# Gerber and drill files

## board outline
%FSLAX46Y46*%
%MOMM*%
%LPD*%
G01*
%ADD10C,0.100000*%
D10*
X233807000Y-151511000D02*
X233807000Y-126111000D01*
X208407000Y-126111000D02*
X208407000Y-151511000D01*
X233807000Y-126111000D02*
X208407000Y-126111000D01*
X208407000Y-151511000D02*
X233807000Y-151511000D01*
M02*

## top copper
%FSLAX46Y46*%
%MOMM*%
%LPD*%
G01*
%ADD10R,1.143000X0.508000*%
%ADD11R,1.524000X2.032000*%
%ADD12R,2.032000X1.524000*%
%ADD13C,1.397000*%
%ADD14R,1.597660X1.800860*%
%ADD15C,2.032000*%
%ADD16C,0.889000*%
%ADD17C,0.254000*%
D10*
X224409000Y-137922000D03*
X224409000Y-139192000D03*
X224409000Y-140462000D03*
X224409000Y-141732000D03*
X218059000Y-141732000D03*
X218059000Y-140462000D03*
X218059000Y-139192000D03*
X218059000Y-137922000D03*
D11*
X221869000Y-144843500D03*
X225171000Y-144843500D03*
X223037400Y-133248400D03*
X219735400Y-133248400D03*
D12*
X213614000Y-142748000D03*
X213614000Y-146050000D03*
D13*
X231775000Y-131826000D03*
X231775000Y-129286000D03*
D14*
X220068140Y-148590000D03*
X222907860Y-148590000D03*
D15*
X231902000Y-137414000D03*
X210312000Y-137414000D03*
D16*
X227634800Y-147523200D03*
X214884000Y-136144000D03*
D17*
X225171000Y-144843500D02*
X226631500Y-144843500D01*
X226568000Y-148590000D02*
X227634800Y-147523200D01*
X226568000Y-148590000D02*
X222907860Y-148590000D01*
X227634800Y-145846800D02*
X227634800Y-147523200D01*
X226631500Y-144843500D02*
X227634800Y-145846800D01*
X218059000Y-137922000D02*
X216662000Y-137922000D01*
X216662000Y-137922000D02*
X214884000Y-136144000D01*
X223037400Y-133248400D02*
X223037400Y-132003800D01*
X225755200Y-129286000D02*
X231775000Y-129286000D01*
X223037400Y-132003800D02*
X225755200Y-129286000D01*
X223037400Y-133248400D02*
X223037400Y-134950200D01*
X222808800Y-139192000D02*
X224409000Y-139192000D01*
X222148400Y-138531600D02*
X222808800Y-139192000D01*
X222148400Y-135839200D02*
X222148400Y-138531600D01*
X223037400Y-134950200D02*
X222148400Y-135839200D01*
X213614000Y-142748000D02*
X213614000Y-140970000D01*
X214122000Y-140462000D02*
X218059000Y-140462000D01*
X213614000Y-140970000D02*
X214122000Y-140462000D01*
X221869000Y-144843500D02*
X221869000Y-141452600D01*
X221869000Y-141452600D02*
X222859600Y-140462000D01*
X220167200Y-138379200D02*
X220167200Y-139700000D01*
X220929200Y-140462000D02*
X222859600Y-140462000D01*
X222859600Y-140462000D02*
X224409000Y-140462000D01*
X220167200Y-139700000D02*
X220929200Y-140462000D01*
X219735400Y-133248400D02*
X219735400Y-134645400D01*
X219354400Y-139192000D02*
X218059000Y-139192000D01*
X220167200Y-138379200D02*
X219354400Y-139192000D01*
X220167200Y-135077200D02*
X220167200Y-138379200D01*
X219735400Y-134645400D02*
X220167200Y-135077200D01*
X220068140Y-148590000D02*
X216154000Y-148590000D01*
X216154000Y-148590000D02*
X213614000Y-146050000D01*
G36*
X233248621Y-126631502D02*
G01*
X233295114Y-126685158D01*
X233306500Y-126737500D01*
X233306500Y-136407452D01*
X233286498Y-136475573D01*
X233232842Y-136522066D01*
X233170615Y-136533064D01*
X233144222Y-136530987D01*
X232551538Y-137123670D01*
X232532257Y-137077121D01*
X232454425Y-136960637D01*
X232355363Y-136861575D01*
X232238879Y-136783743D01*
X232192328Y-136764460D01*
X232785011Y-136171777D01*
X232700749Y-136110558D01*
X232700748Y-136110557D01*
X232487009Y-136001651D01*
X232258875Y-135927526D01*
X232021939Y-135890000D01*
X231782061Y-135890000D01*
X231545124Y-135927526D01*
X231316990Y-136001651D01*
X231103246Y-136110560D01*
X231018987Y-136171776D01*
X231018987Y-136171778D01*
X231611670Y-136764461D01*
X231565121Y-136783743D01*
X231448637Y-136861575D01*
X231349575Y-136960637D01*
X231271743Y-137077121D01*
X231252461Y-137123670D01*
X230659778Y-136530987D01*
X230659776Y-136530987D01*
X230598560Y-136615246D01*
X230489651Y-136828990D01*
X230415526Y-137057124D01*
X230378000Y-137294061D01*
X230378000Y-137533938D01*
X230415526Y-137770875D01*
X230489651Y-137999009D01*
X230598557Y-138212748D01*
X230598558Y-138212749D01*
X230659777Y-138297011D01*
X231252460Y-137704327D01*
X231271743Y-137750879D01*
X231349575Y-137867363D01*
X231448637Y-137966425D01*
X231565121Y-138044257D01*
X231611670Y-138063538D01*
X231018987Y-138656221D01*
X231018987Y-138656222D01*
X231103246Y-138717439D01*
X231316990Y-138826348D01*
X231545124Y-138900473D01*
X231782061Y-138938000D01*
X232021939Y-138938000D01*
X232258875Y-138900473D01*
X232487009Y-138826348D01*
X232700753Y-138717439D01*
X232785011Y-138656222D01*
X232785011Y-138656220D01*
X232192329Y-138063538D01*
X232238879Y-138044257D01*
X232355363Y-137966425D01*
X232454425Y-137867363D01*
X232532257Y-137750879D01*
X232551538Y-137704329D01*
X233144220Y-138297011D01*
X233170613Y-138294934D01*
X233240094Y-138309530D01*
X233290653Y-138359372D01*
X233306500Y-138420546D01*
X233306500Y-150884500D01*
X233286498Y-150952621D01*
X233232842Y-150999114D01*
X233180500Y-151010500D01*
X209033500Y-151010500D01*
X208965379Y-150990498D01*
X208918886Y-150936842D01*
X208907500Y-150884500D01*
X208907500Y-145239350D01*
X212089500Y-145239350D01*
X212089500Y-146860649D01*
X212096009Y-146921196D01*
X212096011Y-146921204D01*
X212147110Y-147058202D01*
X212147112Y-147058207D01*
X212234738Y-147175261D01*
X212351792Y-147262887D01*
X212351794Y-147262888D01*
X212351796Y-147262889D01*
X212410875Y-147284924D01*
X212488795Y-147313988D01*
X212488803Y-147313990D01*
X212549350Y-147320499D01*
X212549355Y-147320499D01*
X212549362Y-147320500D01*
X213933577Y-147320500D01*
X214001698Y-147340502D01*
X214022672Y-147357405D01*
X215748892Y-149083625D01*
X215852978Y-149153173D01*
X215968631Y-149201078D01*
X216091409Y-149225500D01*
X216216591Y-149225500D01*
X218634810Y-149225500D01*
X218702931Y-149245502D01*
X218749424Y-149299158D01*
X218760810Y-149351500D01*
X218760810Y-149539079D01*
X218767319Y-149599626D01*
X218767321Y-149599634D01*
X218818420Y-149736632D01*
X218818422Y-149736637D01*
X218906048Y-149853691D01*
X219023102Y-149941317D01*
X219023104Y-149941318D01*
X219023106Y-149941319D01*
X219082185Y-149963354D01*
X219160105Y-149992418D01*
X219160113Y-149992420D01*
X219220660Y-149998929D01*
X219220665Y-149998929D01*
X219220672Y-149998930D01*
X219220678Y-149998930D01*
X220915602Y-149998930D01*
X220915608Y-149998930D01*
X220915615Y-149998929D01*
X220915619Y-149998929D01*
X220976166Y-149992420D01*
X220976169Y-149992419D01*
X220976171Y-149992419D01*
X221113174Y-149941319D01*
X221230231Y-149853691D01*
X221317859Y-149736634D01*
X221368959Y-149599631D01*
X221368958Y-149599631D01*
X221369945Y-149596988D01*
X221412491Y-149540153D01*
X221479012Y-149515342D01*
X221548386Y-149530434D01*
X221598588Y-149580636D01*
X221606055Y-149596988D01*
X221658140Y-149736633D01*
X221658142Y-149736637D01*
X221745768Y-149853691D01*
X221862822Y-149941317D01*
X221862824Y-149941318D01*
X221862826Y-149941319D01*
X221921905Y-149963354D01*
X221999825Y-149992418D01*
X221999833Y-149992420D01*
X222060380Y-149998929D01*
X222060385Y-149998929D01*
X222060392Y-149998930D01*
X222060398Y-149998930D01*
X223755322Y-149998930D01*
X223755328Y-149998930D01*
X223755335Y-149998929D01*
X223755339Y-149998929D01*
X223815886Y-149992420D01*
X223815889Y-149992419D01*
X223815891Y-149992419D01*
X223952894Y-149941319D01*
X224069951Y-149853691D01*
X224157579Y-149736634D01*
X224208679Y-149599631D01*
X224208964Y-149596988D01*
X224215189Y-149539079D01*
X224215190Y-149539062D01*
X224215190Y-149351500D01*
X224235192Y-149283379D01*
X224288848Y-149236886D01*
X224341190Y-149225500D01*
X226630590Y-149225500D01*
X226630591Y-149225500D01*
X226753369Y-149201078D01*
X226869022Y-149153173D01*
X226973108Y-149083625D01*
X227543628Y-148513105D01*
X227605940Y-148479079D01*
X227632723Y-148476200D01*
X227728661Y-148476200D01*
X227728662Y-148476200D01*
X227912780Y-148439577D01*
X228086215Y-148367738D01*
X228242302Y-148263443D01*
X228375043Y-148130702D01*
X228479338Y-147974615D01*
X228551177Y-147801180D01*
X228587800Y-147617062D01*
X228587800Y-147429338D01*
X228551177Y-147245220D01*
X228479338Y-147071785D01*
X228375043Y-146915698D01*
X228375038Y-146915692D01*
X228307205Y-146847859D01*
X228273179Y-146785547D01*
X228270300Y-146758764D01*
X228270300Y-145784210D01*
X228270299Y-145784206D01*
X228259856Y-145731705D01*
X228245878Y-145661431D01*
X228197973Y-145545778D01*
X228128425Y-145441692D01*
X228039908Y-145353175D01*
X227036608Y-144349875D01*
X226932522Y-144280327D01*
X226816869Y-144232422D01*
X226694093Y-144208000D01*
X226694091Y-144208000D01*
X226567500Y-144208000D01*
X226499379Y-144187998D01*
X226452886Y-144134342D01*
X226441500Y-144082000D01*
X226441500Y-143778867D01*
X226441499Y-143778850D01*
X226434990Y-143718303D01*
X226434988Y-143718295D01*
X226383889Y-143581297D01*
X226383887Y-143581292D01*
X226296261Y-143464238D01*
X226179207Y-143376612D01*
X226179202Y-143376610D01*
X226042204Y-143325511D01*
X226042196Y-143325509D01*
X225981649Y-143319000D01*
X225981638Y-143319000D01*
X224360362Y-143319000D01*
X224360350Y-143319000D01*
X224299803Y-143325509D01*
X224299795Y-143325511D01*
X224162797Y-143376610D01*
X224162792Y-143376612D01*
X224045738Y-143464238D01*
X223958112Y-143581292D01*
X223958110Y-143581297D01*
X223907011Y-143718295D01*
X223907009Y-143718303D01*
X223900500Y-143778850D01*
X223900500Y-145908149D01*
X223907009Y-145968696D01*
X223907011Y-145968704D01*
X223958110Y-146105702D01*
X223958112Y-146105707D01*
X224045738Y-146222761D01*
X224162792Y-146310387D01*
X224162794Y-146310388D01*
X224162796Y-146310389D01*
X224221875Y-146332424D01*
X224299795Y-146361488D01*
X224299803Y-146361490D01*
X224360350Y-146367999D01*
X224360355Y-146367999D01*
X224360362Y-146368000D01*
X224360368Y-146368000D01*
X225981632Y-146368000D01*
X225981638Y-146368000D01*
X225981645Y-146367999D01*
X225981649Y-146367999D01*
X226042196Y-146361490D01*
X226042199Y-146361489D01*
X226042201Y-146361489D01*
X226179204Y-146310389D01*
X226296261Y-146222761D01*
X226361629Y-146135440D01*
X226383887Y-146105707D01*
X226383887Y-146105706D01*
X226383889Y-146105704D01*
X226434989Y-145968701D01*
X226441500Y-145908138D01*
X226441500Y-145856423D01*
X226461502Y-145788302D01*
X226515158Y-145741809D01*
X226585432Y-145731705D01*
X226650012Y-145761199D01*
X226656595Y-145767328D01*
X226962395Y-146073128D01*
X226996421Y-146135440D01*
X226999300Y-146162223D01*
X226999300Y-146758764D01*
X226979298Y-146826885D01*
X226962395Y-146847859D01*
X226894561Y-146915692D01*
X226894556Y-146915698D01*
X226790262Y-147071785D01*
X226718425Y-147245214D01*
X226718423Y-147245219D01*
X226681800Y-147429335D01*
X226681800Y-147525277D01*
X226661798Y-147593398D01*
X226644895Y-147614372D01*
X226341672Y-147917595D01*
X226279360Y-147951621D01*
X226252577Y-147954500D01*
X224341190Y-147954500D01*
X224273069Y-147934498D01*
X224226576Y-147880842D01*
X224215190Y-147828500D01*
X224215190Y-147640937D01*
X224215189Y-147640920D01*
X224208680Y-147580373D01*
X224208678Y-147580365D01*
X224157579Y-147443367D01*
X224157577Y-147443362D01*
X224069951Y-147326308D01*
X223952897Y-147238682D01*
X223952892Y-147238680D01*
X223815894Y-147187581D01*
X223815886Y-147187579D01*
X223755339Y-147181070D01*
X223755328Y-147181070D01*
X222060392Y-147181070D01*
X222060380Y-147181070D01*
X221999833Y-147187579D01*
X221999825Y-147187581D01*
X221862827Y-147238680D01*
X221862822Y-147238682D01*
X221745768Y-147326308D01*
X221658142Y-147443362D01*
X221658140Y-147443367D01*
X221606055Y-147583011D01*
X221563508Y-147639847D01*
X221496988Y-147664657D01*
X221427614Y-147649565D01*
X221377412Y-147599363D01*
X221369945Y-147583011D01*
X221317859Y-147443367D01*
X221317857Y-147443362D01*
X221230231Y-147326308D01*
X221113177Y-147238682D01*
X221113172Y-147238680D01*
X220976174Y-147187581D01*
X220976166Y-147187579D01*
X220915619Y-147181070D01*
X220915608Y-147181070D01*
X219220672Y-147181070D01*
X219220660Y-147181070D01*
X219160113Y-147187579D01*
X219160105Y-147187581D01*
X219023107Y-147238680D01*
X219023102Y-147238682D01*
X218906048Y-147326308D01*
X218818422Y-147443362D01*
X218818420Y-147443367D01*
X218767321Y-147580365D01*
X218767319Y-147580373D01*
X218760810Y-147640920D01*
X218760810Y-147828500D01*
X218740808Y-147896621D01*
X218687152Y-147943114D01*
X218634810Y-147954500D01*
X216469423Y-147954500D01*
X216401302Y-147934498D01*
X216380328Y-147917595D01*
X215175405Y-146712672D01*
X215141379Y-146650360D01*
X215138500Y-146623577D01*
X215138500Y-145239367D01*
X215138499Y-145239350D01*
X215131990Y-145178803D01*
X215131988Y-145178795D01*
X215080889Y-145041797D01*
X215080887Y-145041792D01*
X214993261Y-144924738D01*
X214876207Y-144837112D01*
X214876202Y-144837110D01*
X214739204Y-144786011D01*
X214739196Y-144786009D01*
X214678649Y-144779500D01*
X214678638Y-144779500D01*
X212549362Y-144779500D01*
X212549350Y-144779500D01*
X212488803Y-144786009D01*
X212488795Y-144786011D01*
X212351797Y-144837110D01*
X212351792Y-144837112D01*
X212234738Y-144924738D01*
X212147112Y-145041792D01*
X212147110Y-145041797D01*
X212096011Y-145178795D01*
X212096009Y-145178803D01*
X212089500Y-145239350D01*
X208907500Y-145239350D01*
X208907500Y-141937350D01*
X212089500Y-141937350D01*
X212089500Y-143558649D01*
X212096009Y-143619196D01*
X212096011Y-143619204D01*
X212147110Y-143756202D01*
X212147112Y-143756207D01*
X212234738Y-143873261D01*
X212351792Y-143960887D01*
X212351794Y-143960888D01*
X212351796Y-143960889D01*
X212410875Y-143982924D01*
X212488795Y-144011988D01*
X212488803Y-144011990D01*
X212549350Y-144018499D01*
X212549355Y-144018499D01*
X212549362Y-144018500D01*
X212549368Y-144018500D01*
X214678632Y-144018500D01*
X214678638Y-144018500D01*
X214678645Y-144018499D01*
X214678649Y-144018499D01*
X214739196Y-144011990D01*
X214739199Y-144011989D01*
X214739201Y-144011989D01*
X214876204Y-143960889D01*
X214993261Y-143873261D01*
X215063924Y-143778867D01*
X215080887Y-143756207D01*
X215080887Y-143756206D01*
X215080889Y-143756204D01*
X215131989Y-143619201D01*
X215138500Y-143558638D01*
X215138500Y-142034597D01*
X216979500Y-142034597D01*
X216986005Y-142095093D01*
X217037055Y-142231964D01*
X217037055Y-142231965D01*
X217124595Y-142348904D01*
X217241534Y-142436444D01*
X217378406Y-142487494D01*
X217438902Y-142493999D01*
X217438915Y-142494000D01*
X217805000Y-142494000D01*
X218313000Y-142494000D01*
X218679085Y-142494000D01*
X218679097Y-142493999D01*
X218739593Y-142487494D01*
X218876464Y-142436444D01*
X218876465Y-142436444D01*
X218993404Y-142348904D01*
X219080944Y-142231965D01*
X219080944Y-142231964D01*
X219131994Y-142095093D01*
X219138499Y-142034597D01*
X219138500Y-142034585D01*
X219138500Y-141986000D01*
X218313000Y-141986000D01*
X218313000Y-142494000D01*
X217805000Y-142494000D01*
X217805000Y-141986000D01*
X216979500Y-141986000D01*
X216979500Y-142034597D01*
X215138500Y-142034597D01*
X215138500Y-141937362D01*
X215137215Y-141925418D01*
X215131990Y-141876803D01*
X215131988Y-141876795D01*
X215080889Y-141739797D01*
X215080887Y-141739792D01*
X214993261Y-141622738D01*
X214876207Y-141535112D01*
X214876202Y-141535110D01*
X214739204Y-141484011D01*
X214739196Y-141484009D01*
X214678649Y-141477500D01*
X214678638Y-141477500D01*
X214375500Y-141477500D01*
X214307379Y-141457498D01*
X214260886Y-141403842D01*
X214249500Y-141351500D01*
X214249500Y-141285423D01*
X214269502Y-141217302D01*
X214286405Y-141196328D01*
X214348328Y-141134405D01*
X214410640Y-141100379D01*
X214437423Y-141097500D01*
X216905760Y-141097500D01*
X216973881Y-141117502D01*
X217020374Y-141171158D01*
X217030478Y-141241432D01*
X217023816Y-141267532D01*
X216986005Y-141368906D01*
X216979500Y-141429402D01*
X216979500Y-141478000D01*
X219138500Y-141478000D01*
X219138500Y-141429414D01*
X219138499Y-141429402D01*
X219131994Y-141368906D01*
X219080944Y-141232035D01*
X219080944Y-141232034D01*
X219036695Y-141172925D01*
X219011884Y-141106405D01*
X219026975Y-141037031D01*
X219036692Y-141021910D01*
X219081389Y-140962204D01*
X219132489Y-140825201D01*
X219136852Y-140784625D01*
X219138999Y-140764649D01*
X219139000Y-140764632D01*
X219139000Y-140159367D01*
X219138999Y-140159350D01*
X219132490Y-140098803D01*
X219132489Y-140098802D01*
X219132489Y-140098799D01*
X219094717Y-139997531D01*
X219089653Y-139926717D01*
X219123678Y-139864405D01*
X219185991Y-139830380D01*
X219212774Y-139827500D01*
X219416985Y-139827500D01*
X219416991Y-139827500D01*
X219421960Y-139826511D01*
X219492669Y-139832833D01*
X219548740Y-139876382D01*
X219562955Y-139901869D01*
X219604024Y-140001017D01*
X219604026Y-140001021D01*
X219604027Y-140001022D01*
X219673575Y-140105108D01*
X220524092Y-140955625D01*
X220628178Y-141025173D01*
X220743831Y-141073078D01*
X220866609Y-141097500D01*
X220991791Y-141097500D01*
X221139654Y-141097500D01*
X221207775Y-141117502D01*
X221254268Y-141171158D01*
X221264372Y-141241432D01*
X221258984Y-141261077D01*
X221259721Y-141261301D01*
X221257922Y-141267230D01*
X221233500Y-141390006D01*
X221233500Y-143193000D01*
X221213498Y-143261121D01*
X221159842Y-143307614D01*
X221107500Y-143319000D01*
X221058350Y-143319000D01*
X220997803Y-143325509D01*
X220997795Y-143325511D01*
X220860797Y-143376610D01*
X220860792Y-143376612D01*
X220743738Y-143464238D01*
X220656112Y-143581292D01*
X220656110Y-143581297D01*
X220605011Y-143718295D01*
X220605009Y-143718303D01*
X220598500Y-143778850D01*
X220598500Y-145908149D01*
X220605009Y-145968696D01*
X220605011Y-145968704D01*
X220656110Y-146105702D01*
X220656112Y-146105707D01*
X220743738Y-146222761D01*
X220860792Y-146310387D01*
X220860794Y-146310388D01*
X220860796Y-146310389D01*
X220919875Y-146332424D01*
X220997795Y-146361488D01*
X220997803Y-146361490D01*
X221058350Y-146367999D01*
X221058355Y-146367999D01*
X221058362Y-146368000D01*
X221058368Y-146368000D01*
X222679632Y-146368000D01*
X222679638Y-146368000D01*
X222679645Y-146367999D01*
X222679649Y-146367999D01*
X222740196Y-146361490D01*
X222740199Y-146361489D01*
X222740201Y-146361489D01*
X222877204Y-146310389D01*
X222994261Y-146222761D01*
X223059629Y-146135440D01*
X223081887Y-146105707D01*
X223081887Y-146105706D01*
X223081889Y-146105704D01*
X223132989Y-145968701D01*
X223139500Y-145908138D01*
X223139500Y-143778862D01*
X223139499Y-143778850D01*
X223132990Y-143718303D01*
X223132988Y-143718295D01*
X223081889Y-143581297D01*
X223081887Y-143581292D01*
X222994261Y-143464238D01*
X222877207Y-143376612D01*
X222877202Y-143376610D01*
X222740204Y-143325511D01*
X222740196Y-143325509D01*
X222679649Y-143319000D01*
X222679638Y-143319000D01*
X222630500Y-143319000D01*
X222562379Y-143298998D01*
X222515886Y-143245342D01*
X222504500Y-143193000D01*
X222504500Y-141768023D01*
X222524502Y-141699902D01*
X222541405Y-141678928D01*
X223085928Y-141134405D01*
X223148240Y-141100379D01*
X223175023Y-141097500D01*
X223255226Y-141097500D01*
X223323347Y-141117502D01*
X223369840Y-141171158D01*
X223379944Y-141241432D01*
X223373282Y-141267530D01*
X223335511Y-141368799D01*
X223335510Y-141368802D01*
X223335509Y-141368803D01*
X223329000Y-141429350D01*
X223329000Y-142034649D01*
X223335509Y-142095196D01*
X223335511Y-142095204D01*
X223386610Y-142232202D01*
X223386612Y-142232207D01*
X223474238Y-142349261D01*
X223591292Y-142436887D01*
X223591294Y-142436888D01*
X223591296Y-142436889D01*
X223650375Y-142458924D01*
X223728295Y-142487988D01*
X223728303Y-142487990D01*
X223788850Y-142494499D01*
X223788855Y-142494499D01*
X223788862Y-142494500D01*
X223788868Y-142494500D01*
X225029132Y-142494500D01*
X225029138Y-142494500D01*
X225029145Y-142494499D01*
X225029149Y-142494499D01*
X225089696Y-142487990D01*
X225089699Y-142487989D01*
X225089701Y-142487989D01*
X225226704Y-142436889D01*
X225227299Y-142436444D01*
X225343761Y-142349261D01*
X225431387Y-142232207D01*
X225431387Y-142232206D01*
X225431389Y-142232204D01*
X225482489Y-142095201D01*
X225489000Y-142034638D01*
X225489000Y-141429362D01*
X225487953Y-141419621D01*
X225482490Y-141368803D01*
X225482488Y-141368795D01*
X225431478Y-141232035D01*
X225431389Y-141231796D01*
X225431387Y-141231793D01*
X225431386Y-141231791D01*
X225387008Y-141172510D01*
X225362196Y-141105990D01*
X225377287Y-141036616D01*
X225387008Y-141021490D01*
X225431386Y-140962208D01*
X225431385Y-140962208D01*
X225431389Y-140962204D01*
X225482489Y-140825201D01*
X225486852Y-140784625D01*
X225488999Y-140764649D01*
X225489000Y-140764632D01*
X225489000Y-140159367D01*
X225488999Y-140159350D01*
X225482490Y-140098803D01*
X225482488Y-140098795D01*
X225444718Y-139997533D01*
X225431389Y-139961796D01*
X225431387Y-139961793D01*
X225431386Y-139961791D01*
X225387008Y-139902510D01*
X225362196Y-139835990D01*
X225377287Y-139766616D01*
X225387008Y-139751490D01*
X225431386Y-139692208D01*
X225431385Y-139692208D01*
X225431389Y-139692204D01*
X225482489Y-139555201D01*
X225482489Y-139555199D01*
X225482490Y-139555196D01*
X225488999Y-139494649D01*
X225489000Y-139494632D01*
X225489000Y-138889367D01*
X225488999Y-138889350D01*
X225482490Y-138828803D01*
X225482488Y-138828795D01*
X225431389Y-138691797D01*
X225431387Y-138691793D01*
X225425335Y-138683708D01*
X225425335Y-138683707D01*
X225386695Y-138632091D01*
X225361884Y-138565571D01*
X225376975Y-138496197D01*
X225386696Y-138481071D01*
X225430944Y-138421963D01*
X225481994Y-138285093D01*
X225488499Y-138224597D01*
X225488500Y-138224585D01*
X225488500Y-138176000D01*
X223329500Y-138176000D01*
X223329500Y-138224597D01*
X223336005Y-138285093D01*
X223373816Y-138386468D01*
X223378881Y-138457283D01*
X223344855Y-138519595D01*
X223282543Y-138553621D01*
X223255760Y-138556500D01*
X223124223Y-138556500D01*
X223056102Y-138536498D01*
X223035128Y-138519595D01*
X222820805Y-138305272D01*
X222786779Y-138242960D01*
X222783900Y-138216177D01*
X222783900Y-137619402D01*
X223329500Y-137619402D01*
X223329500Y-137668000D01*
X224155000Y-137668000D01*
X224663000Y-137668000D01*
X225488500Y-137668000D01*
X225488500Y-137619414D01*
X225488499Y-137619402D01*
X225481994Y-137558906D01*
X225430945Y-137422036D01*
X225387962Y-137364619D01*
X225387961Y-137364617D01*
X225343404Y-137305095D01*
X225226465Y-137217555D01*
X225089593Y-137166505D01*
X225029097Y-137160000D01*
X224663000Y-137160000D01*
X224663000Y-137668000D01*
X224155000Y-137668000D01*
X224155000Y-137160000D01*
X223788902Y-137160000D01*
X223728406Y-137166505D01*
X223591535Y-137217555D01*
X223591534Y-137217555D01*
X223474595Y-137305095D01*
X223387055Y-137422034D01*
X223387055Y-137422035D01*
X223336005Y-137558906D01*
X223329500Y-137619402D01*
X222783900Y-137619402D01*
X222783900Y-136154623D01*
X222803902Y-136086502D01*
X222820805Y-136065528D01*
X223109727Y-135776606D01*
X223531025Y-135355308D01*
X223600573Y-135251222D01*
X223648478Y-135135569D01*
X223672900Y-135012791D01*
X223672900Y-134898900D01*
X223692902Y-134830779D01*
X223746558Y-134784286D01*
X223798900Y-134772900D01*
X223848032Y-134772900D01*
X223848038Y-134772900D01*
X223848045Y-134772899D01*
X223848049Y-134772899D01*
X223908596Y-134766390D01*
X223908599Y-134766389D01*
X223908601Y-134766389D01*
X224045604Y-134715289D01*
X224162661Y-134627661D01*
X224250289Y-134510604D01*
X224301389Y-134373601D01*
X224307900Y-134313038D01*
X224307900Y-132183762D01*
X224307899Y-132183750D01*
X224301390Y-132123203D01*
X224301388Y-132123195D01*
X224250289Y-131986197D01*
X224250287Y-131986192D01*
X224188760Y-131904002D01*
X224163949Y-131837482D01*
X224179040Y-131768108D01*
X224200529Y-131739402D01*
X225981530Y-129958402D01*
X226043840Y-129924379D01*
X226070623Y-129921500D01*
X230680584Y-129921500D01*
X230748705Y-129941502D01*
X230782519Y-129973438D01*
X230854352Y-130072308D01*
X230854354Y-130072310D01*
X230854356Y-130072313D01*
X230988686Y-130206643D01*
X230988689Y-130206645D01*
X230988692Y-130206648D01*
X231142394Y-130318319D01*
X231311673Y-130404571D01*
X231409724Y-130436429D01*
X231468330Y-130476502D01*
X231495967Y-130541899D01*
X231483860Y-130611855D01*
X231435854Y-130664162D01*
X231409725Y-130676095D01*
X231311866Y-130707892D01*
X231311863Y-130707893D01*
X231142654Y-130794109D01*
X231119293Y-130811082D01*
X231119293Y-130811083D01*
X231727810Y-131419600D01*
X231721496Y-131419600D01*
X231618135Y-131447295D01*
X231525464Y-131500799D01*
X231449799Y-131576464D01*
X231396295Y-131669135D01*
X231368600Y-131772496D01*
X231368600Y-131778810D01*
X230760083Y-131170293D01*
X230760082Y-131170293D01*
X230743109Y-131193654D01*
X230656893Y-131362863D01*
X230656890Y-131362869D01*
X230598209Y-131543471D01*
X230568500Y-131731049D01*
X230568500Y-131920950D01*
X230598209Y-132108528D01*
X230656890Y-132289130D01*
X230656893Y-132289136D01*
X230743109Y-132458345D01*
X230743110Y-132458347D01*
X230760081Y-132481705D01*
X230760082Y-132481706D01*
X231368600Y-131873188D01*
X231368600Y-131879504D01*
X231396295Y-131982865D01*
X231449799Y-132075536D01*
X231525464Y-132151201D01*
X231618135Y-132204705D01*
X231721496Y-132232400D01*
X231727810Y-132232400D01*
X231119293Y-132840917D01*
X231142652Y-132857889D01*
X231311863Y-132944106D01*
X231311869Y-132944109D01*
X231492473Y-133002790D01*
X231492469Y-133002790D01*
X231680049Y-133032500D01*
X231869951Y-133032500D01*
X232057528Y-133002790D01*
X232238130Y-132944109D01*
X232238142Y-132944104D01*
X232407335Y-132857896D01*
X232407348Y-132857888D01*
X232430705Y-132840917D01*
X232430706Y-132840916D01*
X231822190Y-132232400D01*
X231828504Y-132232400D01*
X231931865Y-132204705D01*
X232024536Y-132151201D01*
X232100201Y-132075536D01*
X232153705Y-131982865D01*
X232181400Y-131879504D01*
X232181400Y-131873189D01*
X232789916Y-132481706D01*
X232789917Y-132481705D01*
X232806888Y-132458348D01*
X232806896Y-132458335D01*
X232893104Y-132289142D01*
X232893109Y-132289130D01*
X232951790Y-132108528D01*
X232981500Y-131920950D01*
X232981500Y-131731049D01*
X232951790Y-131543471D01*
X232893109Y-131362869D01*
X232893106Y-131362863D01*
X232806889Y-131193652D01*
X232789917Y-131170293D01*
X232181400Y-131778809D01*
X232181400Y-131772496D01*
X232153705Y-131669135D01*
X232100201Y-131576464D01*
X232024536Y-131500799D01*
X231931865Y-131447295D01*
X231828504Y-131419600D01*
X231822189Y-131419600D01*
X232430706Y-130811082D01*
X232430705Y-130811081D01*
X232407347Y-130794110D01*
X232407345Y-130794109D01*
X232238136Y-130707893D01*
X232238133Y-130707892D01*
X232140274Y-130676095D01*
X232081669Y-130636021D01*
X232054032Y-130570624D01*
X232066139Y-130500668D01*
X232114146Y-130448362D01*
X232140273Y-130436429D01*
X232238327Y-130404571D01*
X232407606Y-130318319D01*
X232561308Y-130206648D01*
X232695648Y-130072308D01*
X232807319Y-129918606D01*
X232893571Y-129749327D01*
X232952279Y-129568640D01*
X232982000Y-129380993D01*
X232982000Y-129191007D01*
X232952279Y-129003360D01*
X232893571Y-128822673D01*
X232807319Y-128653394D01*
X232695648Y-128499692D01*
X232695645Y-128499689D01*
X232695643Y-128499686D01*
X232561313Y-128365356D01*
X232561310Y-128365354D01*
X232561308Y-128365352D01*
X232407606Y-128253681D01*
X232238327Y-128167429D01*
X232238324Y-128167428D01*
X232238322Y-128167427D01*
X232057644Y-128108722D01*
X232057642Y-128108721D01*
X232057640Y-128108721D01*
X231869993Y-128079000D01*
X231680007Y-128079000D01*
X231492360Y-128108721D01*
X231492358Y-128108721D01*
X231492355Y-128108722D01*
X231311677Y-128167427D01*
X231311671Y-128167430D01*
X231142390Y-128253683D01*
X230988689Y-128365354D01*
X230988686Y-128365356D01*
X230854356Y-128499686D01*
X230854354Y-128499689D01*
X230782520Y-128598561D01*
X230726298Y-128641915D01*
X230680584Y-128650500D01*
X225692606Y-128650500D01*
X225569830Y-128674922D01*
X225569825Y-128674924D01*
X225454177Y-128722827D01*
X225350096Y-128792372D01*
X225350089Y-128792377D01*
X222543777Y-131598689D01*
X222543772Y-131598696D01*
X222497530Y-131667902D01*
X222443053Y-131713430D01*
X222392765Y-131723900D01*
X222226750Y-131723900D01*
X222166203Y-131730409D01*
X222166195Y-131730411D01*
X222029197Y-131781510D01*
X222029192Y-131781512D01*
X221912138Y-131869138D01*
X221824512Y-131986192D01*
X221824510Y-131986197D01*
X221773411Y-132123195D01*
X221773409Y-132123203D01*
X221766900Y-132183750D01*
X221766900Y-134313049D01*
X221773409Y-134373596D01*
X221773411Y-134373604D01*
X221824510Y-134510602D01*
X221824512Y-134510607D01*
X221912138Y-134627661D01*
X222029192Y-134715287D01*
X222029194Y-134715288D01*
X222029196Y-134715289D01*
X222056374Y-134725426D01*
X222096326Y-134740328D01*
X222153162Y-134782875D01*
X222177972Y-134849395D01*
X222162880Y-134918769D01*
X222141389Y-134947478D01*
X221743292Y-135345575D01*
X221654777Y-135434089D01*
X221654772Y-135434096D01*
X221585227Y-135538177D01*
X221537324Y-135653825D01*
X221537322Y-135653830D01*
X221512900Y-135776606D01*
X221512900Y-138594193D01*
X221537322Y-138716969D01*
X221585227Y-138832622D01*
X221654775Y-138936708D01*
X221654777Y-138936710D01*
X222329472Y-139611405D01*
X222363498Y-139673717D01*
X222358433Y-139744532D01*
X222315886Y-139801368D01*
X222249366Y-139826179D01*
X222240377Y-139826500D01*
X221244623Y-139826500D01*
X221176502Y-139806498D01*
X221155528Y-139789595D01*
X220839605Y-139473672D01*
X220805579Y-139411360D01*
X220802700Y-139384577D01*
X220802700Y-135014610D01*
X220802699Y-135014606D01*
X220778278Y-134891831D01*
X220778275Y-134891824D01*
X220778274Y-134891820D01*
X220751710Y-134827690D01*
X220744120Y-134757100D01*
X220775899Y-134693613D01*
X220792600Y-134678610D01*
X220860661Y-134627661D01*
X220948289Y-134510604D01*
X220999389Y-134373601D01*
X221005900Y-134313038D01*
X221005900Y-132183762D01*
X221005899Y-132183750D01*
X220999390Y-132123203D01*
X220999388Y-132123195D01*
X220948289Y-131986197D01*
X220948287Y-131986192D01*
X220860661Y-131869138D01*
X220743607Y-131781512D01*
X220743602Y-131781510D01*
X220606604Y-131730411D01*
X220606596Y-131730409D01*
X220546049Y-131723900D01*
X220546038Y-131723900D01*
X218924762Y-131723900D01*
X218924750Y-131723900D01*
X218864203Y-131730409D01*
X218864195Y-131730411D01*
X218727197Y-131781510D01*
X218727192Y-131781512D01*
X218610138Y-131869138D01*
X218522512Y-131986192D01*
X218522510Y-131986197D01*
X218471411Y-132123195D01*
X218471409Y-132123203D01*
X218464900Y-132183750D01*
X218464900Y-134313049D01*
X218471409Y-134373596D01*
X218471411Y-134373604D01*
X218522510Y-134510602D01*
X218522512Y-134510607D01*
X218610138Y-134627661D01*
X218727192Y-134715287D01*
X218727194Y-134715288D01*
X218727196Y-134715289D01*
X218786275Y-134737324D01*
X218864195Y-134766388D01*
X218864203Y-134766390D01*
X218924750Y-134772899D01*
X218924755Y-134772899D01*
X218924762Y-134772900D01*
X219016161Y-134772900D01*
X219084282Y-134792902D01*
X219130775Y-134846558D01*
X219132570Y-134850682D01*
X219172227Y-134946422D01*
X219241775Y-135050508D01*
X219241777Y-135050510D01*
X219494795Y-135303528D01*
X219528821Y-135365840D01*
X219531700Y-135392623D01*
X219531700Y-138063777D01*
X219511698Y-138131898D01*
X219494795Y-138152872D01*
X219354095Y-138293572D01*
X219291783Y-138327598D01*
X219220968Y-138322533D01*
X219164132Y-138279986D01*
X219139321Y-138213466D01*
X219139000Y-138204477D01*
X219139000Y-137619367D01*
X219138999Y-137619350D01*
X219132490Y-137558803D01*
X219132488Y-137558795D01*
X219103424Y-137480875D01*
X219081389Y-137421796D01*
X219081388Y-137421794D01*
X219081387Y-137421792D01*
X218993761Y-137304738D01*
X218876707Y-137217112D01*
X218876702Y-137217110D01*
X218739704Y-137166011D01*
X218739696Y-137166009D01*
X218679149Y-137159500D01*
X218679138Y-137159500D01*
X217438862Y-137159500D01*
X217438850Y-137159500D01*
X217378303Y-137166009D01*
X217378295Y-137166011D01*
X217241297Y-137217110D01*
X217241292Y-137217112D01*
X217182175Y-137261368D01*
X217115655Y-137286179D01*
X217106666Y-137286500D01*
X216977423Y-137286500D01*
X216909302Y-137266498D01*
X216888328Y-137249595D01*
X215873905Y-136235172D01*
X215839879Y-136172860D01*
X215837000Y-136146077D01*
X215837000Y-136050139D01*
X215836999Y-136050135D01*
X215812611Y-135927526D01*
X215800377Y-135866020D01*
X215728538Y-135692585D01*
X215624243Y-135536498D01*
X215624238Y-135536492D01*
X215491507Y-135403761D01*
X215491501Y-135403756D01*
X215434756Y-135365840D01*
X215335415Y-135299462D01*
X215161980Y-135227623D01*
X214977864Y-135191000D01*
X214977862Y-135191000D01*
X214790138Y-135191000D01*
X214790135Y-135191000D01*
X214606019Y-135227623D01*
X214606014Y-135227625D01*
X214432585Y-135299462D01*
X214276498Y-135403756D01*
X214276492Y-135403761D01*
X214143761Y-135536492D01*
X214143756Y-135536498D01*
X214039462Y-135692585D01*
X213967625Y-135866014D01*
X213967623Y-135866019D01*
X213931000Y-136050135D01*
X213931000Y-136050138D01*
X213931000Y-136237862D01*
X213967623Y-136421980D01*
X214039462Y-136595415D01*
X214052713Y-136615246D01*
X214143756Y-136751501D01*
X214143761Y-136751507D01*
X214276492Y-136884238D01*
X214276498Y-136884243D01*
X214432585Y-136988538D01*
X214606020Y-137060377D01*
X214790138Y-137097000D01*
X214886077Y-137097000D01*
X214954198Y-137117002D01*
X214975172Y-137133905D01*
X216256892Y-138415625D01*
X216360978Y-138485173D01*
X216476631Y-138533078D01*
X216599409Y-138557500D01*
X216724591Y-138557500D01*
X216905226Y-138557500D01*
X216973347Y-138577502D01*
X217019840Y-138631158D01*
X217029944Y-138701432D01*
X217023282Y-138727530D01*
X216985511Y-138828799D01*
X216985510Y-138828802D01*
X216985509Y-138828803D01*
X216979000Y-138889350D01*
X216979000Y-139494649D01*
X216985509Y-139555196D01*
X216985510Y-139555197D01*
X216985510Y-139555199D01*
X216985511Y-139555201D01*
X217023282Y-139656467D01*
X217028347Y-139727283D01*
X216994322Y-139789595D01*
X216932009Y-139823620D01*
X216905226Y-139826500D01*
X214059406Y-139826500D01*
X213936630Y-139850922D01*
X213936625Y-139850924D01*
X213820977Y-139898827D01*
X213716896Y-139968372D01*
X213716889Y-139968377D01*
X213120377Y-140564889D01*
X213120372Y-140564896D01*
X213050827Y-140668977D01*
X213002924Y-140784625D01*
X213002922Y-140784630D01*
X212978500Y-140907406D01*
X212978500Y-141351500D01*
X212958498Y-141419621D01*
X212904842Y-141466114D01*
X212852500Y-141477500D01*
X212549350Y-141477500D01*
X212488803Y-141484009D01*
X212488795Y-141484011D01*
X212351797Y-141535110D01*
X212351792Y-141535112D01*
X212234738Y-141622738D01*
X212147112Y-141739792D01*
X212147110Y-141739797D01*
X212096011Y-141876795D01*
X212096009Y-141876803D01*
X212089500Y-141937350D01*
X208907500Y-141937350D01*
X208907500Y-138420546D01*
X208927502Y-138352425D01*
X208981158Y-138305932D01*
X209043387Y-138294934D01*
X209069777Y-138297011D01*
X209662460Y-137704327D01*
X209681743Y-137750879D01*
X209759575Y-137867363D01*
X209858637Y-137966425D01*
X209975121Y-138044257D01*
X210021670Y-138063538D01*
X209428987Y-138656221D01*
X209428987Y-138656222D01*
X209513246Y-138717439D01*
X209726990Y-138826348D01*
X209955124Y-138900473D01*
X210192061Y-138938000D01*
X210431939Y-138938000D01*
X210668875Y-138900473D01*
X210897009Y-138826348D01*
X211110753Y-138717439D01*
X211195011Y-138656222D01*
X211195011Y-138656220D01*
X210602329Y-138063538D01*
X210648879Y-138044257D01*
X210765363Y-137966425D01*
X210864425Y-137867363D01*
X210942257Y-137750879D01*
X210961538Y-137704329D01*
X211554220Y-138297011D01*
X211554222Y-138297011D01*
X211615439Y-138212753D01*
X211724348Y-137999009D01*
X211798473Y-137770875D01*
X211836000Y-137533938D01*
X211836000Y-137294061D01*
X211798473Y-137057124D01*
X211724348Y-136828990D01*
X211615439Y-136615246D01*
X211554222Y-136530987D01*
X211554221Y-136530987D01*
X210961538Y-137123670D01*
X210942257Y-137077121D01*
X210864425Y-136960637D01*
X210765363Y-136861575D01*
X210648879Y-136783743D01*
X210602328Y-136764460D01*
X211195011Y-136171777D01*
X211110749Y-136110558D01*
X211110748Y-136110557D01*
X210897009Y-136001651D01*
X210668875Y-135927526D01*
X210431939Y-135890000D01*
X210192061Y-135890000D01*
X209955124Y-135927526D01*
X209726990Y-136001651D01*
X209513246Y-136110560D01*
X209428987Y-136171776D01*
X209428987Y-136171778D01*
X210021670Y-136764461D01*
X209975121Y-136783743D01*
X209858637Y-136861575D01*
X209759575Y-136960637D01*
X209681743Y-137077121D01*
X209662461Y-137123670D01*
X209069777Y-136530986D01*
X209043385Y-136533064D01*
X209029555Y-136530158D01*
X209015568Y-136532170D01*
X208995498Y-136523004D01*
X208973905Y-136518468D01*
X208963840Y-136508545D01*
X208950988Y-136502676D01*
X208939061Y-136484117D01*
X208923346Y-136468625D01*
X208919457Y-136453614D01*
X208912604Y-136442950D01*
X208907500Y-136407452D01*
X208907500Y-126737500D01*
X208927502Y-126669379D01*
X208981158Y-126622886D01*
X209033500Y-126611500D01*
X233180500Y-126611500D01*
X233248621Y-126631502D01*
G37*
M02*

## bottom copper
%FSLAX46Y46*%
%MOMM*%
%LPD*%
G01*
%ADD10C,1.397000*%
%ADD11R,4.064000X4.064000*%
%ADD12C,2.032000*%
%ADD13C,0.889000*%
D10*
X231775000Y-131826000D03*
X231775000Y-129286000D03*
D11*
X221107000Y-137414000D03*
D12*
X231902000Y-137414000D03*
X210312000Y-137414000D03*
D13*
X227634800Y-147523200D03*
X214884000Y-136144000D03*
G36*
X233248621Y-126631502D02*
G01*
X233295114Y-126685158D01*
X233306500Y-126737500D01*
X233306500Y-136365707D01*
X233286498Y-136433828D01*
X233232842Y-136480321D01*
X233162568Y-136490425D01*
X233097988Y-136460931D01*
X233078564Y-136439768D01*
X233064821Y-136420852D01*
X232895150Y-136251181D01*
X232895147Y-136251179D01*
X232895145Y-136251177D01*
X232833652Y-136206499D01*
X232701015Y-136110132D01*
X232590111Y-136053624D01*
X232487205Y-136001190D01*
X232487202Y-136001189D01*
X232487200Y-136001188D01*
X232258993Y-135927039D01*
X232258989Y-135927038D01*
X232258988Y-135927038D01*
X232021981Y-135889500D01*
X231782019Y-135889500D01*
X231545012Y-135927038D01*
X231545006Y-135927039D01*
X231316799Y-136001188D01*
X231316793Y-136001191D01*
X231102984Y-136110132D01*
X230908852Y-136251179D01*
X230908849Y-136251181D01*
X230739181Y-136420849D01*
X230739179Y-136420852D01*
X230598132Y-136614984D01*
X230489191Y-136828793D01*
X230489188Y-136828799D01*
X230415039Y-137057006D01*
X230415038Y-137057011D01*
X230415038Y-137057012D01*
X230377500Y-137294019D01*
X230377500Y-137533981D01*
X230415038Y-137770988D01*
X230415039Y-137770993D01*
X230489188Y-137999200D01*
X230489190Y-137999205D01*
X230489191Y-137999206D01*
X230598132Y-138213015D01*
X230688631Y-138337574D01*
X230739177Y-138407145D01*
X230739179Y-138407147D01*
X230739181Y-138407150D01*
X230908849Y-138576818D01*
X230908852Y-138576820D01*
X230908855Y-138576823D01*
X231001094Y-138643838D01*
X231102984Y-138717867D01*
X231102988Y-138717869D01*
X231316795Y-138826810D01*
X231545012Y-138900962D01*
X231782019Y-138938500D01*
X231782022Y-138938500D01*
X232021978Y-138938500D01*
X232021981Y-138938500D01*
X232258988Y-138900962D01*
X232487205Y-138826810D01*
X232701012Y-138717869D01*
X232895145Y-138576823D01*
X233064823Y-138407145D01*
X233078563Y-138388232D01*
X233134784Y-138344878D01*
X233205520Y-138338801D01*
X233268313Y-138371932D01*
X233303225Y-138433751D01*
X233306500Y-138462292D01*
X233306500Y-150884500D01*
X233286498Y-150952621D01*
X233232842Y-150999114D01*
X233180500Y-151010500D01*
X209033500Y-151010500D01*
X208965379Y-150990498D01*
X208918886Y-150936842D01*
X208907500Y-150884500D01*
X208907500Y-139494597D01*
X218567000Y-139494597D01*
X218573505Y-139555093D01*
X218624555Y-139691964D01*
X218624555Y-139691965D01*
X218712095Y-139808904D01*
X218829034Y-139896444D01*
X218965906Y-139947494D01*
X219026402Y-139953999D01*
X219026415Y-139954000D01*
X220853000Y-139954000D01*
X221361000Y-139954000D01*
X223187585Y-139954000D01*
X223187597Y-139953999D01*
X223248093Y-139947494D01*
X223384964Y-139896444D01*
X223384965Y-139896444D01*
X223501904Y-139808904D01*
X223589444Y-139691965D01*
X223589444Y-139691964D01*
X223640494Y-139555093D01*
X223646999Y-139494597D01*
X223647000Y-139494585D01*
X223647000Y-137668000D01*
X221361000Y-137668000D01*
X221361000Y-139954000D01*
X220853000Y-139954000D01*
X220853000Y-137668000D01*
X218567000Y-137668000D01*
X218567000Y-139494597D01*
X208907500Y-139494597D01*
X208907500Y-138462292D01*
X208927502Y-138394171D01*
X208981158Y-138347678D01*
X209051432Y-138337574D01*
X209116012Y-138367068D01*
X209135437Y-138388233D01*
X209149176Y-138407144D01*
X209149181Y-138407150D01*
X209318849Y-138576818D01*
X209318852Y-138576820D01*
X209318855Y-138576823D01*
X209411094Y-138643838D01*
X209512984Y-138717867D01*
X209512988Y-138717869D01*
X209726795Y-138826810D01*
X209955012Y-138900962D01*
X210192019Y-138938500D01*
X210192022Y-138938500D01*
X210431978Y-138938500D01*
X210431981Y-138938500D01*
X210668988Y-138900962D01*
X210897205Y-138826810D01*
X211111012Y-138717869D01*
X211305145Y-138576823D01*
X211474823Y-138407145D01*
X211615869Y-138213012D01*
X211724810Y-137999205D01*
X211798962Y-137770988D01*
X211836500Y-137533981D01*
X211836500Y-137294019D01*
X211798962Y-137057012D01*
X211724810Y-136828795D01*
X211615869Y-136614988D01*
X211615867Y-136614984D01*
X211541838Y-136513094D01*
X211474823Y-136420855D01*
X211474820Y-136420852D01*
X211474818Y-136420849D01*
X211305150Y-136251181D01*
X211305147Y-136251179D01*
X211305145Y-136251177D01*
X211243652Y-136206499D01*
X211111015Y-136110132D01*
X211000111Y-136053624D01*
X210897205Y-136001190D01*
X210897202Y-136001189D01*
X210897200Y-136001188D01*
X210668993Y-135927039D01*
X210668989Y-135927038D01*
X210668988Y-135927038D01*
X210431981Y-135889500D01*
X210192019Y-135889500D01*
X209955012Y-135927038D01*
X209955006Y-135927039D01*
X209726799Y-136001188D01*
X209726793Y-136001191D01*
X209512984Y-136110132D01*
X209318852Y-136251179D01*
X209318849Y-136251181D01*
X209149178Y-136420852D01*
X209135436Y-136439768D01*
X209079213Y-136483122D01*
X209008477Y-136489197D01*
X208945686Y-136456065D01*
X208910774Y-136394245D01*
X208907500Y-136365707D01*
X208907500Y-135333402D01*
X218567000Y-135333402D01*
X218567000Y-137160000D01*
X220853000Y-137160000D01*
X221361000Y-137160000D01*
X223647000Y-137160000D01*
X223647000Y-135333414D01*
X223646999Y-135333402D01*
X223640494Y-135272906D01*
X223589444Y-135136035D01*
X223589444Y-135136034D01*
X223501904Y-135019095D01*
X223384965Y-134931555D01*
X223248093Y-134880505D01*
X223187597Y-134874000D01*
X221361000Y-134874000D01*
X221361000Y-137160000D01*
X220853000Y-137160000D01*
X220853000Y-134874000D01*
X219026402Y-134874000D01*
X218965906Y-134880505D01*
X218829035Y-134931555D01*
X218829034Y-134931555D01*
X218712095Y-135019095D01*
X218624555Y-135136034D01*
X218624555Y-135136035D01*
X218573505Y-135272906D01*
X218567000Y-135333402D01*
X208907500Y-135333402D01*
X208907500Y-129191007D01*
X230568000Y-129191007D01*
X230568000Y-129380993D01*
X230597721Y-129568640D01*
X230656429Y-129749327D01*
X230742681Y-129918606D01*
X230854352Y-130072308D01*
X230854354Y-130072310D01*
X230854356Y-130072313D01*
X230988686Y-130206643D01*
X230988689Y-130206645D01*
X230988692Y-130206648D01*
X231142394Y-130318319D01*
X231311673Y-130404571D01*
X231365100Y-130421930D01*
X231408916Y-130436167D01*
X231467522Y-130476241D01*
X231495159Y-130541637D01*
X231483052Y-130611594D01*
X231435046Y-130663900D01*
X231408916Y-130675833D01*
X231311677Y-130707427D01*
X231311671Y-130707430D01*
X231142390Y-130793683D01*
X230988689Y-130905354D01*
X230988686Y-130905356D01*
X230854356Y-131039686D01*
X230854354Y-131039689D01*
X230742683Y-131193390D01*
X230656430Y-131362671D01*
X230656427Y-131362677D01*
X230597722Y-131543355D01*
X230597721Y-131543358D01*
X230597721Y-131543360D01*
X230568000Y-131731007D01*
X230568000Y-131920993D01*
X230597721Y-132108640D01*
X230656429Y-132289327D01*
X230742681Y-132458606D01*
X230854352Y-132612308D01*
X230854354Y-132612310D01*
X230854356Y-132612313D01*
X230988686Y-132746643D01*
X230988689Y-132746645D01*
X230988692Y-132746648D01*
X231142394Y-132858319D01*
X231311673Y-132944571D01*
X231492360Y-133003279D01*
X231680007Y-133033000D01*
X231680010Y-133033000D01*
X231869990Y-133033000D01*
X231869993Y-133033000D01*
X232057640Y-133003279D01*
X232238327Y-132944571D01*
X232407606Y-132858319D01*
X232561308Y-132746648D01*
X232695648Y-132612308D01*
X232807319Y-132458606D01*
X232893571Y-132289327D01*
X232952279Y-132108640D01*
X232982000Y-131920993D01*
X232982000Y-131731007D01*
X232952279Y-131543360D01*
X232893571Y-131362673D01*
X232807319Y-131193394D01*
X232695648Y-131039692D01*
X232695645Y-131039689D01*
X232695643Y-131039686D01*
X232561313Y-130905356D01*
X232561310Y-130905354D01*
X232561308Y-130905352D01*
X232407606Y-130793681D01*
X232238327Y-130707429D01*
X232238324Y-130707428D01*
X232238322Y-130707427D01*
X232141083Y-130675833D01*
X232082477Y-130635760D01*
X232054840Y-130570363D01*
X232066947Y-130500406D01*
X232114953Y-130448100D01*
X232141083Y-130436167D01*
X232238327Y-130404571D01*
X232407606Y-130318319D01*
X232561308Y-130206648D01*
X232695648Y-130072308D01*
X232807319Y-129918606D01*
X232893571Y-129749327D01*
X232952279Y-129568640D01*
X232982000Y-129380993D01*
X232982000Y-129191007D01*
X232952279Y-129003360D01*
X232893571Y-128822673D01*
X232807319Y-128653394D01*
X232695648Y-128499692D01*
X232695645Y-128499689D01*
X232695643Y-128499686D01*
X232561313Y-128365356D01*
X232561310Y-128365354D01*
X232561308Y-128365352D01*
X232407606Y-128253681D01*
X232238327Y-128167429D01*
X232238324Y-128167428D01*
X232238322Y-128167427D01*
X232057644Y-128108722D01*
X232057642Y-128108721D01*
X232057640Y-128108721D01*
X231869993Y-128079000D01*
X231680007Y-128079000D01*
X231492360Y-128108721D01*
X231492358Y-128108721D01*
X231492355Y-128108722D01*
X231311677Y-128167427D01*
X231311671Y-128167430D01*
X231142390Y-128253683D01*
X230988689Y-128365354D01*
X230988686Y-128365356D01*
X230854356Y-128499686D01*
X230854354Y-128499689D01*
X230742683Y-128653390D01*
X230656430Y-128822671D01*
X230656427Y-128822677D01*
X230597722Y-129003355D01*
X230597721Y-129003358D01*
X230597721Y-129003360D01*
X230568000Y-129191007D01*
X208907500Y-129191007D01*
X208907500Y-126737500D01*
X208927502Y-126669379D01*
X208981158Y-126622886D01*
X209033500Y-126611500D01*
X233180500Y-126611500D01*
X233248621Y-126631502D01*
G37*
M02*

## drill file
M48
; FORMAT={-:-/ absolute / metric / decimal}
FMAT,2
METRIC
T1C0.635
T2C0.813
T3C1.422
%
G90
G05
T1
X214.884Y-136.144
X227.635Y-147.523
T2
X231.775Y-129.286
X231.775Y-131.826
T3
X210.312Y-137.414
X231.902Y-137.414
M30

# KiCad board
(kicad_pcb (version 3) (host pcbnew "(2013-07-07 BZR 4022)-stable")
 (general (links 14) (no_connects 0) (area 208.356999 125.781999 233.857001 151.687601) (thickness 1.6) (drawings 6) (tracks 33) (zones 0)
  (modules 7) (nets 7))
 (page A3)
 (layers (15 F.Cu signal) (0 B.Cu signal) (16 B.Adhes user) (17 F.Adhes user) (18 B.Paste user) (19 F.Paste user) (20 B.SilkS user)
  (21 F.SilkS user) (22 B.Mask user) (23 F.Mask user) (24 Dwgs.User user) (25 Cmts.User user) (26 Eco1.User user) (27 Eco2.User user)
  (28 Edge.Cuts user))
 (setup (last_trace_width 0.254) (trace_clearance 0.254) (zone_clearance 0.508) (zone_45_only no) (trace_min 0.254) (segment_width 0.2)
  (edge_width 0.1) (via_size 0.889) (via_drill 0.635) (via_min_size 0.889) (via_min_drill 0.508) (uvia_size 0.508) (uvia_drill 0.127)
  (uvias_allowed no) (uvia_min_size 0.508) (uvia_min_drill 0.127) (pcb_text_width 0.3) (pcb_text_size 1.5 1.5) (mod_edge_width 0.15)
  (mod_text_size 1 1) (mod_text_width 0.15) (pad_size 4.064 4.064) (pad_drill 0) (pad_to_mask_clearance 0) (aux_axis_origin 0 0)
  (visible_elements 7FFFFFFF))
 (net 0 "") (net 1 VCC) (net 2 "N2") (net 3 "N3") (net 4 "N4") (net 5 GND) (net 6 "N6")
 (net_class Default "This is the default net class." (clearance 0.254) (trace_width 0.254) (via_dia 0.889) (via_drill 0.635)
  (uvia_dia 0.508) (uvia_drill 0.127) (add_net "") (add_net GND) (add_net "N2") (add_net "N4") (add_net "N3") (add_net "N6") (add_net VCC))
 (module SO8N (layer F.Cu) (at 221.234 139.827 270)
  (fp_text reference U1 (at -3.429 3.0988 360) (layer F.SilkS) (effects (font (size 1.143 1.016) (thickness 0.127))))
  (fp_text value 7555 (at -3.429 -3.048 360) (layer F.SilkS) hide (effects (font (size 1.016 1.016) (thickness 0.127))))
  (pad 8 smd rect (at -1.905 -3.175 270) (size 0.508 1.143) (layers F.Cu F.Paste F.Mask) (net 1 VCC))
  (pad 7 smd rect (at -0.635 -3.175 270) (size 0.508 1.143) (layers F.Cu F.Paste F.Mask) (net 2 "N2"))
  (pad 6 smd rect (at 0.635 -3.175 270) (size 0.508 1.143) (layers F.Cu F.Paste F.Mask) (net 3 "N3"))
  (pad 5 smd rect (at 1.905 -3.175 270) (size 0.508 1.143) (layers F.Cu F.Paste F.Mask))
  (pad 4 smd rect (at 1.905 3.175 270) (size 0.508 1.143) (layers F.Cu F.Paste F.Mask) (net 1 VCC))
  (pad 3 smd rect (at 0.635 3.175 270) (size 0.508 1.143) (layers F.Cu F.Paste F.Mask) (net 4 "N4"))
  (pad 2 smd rect (at -0.635 3.175 270) (size 0.508 1.143) (layers F.Cu F.Paste F.Mask) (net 3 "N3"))
  (pad 1 smd rect (at -1.905 3.175 270) (size 0.508 1.143) (layers F.Cu F.Paste F.Mask) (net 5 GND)))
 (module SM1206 (layer F.Cu) (at 223.52 144.8435)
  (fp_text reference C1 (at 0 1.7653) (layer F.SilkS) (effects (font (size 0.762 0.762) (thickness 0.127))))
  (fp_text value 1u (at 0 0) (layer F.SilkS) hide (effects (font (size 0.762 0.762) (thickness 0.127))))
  (pad 1 smd rect (at -1.651 0) (size 1.524 2.032) (layers F.Cu F.Paste F.Mask) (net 3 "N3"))
  (pad 2 smd rect (at 1.651 0) (size 1.524 2.032) (layers F.Cu F.Paste F.Mask) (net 5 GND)))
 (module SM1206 (layer F.Cu) (at 221.3864 133.2484 180)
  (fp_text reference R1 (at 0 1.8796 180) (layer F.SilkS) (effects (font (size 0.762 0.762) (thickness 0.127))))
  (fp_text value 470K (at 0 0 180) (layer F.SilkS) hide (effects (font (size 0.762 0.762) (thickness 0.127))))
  (pad 1 smd rect (at -1.651 0 180) (size 1.524 2.032) (layers F.Cu F.Paste F.Mask) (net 2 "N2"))
  (pad 2 smd rect (at 1.651 0 180) (size 1.524 2.032) (layers F.Cu F.Paste F.Mask) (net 3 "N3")))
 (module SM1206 (layer F.Cu) (at 213.614 144.399 270)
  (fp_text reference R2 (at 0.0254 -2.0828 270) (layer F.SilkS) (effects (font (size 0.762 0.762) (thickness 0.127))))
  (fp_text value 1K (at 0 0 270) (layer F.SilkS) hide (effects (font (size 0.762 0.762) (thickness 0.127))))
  (pad 1 smd rect (at -1.651 0 270) (size 1.524 2.032) (layers F.Cu F.Paste F.Mask) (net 4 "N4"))
  (pad 2 smd rect (at 1.651 0 270) (size 1.524 2.032) (layers F.Cu F.Paste F.Mask) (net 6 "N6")))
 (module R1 (layer F.Cu) (at 231.775 130.556 90) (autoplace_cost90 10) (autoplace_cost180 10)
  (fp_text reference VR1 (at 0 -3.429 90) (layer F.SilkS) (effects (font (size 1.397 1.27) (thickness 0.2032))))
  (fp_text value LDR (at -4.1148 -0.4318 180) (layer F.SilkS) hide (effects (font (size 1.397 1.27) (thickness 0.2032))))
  (pad 1 thru_hole circle (at -1.27 0 90) (size 1.397 1.397) (drill 0.8128) (layers *.Cu *.Mask F.SilkS) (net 1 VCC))
  (pad 2 thru_hole circle (at 1.27 0 90) (size 1.397 1.397) (drill 0.8128) (layers *.Cu *.Mask F.SilkS) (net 2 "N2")))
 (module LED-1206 (layer F.Cu) (at 221.488 148.59)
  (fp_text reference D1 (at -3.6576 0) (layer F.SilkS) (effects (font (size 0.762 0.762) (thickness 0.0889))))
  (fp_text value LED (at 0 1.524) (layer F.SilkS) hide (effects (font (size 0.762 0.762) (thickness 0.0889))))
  (pad 1 smd rect (at -1.41986 0) (size 1.59766 1.80086) (layers F.Cu F.Paste F.Mask) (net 6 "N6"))
  (pad 2 smd rect (at 1.41986 0) (size 1.59766 1.80086) (layers F.Cu F.Paste F.Mask) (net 5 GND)))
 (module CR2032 (layer B.Cu) (at 221.107 137.414 180)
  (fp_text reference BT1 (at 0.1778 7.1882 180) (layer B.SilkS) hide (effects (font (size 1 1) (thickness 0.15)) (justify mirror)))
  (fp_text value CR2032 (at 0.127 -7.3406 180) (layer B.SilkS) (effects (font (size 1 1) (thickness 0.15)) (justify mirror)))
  (pad 2 smd rect (at 0 0 180) (size 4.064 4.064) (layers B.Cu B.Paste B.Mask) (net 5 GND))
  (pad 1 thru_hole circle (at -10.795 0 180) (size 2.032 2.032) (drill 1.4224) (layers *.Cu *.Mask B.SilkS) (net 1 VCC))
  (pad 1 thru_hole circle (at 10.795 0 180) (size 2.032 2.032) (drill 1.4224) (layers *.Cu *.Mask B.SilkS) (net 1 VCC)))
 (gr_line (start 233.807 151.511) (end 233.807 126.111) (angle 90) (layer Edge.Cuts) (width 0.1))
 (gr_line (start 208.407 126.111) (end 208.407 151.511) (angle 90) (layer Edge.Cuts) (width 0.1))
 (gr_line (start 233.807 126.111) (end 208.407 126.111) (angle 90) (layer Edge.Cuts) (width 0.1))
 (gr_line (start 208.407 151.511) (end 233.807 151.511) (angle 90) (layer Edge.Cuts) (width 0.1))
 (segment (start 225.171 144.8435) (end 226.6315 144.8435) (width 0.254) (layer F.Cu) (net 5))
 (segment (start 226.568 148.59) (end 227.6348 147.5232) (width 0.254) (layer F.Cu) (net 5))
 (via (at 227.6348 147.5232) (size 0.889) (layers F.Cu B.Cu) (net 5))
 (segment (start 226.568 148.59) (end 222.90786 148.59) (width 0.254) (layer F.Cu) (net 5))
 (segment (start 227.6348 145.8468) (end 227.6348 147.5232) (width 0.254) (layer F.Cu) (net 5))
 (segment (start 226.6315 144.8435) (end 227.6348 145.8468) (width 0.254) (layer F.Cu) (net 5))
 (segment (start 218.059 137.922) (end 216.662 137.922) (width 0.254) (layer F.Cu) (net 5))
 (via (at 214.884 136.144) (size 0.889) (layers F.Cu B.Cu) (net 5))
 (segment (start 216.662 137.922) (end 214.884 136.144) (width 0.254) (layer F.Cu) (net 5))
 (segment (start 223.0374 133.2484) (end 223.0374 132.0038) (width 0.254) (layer F.Cu) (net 2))
 (segment (start 225.7552 129.286) (end 231.775 129.286) (width 0.254) (layer F.Cu) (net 2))
 (segment (start 223.0374 132.0038) (end 225.7552 129.286) (width 0.254) (layer F.Cu) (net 2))
 (segment (start 223.0374 133.2484) (end 223.0374 134.9502) (width 0.254) (layer F.Cu) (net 2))
 (segment (start 222.8088 139.192) (end 224.409 139.192) (width 0.254) (layer F.Cu) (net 2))
 (segment (start 222.1484 138.5316) (end 222.8088 139.192) (width 0.254) (layer F.Cu) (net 2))
 (segment (start 222.1484 135.8392) (end 222.1484 138.5316) (width 0.254) (layer F.Cu) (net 2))
 (segment (start 223.0374 134.9502) (end 222.1484 135.8392) (width 0.254) (layer F.Cu) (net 2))
 (segment (start 213.614 142.748) (end 213.614 140.97) (width 0.254) (layer F.Cu) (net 4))
 (segment (start 214.122 140.462) (end 218.059 140.462) (width 0.254) (layer F.Cu) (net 4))
 (segment (start 213.614 140.97) (end 214.122 140.462) (width 0.254) (layer F.Cu) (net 4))
 (segment (start 221.869 144.8435) (end 221.869 141.4526) (width 0.254) (layer F.Cu) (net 3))
 (segment (start 221.869 141.4526) (end 222.8596 140.462) (width 0.254) (layer F.Cu) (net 3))
 (segment (start 220.1672 138.3792) (end 220.1672 139.7) (width 0.254) (layer F.Cu) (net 3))
 (segment (start 220.9292 140.462) (end 222.8596 140.462) (width 0.254) (layer F.Cu) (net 3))
 (segment (start 222.8596 140.462) (end 224.409 140.462) (width 0.254) (layer F.Cu) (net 3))
 (segment (start 220.1672 139.7) (end 220.9292 140.462) (width 0.254) (layer F.Cu) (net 3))
 (segment (start 219.7354 133.2484) (end 219.7354 134.6454) (width 0.254) (layer F.Cu) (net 3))
 (segment (start 219.3544 139.192) (end 218.059 139.192) (width 0.254) (layer F.Cu) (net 3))
 (segment (start 220.1672 138.3792) (end 219.3544 139.192) (width 0.254) (layer F.Cu) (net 3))
 (segment (start 220.1672 135.0772) (end 220.1672 138.3792) (width 0.254) (layer F.Cu) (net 3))
 (segment (start 219.7354 134.6454) (end 220.1672 135.0772) (width 0.254) (layer F.Cu) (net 3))
 (segment (start 220.06814 148.59) (end 216.154 148.59) (width 0.254) (layer F.Cu) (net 6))
 (segment (start 216.154 148.59) (end 213.614 146.05) (width 0.254) (layer F.Cu) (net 6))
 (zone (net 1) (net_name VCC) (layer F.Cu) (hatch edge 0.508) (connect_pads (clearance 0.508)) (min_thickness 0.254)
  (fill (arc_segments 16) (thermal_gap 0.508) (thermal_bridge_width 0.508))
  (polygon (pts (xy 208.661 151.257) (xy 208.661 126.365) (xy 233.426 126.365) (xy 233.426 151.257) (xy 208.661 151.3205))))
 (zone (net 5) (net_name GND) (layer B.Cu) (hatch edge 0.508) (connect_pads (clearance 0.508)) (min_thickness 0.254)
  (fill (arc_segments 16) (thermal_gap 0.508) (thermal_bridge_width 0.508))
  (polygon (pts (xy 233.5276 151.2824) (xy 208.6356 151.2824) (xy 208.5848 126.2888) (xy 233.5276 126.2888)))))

